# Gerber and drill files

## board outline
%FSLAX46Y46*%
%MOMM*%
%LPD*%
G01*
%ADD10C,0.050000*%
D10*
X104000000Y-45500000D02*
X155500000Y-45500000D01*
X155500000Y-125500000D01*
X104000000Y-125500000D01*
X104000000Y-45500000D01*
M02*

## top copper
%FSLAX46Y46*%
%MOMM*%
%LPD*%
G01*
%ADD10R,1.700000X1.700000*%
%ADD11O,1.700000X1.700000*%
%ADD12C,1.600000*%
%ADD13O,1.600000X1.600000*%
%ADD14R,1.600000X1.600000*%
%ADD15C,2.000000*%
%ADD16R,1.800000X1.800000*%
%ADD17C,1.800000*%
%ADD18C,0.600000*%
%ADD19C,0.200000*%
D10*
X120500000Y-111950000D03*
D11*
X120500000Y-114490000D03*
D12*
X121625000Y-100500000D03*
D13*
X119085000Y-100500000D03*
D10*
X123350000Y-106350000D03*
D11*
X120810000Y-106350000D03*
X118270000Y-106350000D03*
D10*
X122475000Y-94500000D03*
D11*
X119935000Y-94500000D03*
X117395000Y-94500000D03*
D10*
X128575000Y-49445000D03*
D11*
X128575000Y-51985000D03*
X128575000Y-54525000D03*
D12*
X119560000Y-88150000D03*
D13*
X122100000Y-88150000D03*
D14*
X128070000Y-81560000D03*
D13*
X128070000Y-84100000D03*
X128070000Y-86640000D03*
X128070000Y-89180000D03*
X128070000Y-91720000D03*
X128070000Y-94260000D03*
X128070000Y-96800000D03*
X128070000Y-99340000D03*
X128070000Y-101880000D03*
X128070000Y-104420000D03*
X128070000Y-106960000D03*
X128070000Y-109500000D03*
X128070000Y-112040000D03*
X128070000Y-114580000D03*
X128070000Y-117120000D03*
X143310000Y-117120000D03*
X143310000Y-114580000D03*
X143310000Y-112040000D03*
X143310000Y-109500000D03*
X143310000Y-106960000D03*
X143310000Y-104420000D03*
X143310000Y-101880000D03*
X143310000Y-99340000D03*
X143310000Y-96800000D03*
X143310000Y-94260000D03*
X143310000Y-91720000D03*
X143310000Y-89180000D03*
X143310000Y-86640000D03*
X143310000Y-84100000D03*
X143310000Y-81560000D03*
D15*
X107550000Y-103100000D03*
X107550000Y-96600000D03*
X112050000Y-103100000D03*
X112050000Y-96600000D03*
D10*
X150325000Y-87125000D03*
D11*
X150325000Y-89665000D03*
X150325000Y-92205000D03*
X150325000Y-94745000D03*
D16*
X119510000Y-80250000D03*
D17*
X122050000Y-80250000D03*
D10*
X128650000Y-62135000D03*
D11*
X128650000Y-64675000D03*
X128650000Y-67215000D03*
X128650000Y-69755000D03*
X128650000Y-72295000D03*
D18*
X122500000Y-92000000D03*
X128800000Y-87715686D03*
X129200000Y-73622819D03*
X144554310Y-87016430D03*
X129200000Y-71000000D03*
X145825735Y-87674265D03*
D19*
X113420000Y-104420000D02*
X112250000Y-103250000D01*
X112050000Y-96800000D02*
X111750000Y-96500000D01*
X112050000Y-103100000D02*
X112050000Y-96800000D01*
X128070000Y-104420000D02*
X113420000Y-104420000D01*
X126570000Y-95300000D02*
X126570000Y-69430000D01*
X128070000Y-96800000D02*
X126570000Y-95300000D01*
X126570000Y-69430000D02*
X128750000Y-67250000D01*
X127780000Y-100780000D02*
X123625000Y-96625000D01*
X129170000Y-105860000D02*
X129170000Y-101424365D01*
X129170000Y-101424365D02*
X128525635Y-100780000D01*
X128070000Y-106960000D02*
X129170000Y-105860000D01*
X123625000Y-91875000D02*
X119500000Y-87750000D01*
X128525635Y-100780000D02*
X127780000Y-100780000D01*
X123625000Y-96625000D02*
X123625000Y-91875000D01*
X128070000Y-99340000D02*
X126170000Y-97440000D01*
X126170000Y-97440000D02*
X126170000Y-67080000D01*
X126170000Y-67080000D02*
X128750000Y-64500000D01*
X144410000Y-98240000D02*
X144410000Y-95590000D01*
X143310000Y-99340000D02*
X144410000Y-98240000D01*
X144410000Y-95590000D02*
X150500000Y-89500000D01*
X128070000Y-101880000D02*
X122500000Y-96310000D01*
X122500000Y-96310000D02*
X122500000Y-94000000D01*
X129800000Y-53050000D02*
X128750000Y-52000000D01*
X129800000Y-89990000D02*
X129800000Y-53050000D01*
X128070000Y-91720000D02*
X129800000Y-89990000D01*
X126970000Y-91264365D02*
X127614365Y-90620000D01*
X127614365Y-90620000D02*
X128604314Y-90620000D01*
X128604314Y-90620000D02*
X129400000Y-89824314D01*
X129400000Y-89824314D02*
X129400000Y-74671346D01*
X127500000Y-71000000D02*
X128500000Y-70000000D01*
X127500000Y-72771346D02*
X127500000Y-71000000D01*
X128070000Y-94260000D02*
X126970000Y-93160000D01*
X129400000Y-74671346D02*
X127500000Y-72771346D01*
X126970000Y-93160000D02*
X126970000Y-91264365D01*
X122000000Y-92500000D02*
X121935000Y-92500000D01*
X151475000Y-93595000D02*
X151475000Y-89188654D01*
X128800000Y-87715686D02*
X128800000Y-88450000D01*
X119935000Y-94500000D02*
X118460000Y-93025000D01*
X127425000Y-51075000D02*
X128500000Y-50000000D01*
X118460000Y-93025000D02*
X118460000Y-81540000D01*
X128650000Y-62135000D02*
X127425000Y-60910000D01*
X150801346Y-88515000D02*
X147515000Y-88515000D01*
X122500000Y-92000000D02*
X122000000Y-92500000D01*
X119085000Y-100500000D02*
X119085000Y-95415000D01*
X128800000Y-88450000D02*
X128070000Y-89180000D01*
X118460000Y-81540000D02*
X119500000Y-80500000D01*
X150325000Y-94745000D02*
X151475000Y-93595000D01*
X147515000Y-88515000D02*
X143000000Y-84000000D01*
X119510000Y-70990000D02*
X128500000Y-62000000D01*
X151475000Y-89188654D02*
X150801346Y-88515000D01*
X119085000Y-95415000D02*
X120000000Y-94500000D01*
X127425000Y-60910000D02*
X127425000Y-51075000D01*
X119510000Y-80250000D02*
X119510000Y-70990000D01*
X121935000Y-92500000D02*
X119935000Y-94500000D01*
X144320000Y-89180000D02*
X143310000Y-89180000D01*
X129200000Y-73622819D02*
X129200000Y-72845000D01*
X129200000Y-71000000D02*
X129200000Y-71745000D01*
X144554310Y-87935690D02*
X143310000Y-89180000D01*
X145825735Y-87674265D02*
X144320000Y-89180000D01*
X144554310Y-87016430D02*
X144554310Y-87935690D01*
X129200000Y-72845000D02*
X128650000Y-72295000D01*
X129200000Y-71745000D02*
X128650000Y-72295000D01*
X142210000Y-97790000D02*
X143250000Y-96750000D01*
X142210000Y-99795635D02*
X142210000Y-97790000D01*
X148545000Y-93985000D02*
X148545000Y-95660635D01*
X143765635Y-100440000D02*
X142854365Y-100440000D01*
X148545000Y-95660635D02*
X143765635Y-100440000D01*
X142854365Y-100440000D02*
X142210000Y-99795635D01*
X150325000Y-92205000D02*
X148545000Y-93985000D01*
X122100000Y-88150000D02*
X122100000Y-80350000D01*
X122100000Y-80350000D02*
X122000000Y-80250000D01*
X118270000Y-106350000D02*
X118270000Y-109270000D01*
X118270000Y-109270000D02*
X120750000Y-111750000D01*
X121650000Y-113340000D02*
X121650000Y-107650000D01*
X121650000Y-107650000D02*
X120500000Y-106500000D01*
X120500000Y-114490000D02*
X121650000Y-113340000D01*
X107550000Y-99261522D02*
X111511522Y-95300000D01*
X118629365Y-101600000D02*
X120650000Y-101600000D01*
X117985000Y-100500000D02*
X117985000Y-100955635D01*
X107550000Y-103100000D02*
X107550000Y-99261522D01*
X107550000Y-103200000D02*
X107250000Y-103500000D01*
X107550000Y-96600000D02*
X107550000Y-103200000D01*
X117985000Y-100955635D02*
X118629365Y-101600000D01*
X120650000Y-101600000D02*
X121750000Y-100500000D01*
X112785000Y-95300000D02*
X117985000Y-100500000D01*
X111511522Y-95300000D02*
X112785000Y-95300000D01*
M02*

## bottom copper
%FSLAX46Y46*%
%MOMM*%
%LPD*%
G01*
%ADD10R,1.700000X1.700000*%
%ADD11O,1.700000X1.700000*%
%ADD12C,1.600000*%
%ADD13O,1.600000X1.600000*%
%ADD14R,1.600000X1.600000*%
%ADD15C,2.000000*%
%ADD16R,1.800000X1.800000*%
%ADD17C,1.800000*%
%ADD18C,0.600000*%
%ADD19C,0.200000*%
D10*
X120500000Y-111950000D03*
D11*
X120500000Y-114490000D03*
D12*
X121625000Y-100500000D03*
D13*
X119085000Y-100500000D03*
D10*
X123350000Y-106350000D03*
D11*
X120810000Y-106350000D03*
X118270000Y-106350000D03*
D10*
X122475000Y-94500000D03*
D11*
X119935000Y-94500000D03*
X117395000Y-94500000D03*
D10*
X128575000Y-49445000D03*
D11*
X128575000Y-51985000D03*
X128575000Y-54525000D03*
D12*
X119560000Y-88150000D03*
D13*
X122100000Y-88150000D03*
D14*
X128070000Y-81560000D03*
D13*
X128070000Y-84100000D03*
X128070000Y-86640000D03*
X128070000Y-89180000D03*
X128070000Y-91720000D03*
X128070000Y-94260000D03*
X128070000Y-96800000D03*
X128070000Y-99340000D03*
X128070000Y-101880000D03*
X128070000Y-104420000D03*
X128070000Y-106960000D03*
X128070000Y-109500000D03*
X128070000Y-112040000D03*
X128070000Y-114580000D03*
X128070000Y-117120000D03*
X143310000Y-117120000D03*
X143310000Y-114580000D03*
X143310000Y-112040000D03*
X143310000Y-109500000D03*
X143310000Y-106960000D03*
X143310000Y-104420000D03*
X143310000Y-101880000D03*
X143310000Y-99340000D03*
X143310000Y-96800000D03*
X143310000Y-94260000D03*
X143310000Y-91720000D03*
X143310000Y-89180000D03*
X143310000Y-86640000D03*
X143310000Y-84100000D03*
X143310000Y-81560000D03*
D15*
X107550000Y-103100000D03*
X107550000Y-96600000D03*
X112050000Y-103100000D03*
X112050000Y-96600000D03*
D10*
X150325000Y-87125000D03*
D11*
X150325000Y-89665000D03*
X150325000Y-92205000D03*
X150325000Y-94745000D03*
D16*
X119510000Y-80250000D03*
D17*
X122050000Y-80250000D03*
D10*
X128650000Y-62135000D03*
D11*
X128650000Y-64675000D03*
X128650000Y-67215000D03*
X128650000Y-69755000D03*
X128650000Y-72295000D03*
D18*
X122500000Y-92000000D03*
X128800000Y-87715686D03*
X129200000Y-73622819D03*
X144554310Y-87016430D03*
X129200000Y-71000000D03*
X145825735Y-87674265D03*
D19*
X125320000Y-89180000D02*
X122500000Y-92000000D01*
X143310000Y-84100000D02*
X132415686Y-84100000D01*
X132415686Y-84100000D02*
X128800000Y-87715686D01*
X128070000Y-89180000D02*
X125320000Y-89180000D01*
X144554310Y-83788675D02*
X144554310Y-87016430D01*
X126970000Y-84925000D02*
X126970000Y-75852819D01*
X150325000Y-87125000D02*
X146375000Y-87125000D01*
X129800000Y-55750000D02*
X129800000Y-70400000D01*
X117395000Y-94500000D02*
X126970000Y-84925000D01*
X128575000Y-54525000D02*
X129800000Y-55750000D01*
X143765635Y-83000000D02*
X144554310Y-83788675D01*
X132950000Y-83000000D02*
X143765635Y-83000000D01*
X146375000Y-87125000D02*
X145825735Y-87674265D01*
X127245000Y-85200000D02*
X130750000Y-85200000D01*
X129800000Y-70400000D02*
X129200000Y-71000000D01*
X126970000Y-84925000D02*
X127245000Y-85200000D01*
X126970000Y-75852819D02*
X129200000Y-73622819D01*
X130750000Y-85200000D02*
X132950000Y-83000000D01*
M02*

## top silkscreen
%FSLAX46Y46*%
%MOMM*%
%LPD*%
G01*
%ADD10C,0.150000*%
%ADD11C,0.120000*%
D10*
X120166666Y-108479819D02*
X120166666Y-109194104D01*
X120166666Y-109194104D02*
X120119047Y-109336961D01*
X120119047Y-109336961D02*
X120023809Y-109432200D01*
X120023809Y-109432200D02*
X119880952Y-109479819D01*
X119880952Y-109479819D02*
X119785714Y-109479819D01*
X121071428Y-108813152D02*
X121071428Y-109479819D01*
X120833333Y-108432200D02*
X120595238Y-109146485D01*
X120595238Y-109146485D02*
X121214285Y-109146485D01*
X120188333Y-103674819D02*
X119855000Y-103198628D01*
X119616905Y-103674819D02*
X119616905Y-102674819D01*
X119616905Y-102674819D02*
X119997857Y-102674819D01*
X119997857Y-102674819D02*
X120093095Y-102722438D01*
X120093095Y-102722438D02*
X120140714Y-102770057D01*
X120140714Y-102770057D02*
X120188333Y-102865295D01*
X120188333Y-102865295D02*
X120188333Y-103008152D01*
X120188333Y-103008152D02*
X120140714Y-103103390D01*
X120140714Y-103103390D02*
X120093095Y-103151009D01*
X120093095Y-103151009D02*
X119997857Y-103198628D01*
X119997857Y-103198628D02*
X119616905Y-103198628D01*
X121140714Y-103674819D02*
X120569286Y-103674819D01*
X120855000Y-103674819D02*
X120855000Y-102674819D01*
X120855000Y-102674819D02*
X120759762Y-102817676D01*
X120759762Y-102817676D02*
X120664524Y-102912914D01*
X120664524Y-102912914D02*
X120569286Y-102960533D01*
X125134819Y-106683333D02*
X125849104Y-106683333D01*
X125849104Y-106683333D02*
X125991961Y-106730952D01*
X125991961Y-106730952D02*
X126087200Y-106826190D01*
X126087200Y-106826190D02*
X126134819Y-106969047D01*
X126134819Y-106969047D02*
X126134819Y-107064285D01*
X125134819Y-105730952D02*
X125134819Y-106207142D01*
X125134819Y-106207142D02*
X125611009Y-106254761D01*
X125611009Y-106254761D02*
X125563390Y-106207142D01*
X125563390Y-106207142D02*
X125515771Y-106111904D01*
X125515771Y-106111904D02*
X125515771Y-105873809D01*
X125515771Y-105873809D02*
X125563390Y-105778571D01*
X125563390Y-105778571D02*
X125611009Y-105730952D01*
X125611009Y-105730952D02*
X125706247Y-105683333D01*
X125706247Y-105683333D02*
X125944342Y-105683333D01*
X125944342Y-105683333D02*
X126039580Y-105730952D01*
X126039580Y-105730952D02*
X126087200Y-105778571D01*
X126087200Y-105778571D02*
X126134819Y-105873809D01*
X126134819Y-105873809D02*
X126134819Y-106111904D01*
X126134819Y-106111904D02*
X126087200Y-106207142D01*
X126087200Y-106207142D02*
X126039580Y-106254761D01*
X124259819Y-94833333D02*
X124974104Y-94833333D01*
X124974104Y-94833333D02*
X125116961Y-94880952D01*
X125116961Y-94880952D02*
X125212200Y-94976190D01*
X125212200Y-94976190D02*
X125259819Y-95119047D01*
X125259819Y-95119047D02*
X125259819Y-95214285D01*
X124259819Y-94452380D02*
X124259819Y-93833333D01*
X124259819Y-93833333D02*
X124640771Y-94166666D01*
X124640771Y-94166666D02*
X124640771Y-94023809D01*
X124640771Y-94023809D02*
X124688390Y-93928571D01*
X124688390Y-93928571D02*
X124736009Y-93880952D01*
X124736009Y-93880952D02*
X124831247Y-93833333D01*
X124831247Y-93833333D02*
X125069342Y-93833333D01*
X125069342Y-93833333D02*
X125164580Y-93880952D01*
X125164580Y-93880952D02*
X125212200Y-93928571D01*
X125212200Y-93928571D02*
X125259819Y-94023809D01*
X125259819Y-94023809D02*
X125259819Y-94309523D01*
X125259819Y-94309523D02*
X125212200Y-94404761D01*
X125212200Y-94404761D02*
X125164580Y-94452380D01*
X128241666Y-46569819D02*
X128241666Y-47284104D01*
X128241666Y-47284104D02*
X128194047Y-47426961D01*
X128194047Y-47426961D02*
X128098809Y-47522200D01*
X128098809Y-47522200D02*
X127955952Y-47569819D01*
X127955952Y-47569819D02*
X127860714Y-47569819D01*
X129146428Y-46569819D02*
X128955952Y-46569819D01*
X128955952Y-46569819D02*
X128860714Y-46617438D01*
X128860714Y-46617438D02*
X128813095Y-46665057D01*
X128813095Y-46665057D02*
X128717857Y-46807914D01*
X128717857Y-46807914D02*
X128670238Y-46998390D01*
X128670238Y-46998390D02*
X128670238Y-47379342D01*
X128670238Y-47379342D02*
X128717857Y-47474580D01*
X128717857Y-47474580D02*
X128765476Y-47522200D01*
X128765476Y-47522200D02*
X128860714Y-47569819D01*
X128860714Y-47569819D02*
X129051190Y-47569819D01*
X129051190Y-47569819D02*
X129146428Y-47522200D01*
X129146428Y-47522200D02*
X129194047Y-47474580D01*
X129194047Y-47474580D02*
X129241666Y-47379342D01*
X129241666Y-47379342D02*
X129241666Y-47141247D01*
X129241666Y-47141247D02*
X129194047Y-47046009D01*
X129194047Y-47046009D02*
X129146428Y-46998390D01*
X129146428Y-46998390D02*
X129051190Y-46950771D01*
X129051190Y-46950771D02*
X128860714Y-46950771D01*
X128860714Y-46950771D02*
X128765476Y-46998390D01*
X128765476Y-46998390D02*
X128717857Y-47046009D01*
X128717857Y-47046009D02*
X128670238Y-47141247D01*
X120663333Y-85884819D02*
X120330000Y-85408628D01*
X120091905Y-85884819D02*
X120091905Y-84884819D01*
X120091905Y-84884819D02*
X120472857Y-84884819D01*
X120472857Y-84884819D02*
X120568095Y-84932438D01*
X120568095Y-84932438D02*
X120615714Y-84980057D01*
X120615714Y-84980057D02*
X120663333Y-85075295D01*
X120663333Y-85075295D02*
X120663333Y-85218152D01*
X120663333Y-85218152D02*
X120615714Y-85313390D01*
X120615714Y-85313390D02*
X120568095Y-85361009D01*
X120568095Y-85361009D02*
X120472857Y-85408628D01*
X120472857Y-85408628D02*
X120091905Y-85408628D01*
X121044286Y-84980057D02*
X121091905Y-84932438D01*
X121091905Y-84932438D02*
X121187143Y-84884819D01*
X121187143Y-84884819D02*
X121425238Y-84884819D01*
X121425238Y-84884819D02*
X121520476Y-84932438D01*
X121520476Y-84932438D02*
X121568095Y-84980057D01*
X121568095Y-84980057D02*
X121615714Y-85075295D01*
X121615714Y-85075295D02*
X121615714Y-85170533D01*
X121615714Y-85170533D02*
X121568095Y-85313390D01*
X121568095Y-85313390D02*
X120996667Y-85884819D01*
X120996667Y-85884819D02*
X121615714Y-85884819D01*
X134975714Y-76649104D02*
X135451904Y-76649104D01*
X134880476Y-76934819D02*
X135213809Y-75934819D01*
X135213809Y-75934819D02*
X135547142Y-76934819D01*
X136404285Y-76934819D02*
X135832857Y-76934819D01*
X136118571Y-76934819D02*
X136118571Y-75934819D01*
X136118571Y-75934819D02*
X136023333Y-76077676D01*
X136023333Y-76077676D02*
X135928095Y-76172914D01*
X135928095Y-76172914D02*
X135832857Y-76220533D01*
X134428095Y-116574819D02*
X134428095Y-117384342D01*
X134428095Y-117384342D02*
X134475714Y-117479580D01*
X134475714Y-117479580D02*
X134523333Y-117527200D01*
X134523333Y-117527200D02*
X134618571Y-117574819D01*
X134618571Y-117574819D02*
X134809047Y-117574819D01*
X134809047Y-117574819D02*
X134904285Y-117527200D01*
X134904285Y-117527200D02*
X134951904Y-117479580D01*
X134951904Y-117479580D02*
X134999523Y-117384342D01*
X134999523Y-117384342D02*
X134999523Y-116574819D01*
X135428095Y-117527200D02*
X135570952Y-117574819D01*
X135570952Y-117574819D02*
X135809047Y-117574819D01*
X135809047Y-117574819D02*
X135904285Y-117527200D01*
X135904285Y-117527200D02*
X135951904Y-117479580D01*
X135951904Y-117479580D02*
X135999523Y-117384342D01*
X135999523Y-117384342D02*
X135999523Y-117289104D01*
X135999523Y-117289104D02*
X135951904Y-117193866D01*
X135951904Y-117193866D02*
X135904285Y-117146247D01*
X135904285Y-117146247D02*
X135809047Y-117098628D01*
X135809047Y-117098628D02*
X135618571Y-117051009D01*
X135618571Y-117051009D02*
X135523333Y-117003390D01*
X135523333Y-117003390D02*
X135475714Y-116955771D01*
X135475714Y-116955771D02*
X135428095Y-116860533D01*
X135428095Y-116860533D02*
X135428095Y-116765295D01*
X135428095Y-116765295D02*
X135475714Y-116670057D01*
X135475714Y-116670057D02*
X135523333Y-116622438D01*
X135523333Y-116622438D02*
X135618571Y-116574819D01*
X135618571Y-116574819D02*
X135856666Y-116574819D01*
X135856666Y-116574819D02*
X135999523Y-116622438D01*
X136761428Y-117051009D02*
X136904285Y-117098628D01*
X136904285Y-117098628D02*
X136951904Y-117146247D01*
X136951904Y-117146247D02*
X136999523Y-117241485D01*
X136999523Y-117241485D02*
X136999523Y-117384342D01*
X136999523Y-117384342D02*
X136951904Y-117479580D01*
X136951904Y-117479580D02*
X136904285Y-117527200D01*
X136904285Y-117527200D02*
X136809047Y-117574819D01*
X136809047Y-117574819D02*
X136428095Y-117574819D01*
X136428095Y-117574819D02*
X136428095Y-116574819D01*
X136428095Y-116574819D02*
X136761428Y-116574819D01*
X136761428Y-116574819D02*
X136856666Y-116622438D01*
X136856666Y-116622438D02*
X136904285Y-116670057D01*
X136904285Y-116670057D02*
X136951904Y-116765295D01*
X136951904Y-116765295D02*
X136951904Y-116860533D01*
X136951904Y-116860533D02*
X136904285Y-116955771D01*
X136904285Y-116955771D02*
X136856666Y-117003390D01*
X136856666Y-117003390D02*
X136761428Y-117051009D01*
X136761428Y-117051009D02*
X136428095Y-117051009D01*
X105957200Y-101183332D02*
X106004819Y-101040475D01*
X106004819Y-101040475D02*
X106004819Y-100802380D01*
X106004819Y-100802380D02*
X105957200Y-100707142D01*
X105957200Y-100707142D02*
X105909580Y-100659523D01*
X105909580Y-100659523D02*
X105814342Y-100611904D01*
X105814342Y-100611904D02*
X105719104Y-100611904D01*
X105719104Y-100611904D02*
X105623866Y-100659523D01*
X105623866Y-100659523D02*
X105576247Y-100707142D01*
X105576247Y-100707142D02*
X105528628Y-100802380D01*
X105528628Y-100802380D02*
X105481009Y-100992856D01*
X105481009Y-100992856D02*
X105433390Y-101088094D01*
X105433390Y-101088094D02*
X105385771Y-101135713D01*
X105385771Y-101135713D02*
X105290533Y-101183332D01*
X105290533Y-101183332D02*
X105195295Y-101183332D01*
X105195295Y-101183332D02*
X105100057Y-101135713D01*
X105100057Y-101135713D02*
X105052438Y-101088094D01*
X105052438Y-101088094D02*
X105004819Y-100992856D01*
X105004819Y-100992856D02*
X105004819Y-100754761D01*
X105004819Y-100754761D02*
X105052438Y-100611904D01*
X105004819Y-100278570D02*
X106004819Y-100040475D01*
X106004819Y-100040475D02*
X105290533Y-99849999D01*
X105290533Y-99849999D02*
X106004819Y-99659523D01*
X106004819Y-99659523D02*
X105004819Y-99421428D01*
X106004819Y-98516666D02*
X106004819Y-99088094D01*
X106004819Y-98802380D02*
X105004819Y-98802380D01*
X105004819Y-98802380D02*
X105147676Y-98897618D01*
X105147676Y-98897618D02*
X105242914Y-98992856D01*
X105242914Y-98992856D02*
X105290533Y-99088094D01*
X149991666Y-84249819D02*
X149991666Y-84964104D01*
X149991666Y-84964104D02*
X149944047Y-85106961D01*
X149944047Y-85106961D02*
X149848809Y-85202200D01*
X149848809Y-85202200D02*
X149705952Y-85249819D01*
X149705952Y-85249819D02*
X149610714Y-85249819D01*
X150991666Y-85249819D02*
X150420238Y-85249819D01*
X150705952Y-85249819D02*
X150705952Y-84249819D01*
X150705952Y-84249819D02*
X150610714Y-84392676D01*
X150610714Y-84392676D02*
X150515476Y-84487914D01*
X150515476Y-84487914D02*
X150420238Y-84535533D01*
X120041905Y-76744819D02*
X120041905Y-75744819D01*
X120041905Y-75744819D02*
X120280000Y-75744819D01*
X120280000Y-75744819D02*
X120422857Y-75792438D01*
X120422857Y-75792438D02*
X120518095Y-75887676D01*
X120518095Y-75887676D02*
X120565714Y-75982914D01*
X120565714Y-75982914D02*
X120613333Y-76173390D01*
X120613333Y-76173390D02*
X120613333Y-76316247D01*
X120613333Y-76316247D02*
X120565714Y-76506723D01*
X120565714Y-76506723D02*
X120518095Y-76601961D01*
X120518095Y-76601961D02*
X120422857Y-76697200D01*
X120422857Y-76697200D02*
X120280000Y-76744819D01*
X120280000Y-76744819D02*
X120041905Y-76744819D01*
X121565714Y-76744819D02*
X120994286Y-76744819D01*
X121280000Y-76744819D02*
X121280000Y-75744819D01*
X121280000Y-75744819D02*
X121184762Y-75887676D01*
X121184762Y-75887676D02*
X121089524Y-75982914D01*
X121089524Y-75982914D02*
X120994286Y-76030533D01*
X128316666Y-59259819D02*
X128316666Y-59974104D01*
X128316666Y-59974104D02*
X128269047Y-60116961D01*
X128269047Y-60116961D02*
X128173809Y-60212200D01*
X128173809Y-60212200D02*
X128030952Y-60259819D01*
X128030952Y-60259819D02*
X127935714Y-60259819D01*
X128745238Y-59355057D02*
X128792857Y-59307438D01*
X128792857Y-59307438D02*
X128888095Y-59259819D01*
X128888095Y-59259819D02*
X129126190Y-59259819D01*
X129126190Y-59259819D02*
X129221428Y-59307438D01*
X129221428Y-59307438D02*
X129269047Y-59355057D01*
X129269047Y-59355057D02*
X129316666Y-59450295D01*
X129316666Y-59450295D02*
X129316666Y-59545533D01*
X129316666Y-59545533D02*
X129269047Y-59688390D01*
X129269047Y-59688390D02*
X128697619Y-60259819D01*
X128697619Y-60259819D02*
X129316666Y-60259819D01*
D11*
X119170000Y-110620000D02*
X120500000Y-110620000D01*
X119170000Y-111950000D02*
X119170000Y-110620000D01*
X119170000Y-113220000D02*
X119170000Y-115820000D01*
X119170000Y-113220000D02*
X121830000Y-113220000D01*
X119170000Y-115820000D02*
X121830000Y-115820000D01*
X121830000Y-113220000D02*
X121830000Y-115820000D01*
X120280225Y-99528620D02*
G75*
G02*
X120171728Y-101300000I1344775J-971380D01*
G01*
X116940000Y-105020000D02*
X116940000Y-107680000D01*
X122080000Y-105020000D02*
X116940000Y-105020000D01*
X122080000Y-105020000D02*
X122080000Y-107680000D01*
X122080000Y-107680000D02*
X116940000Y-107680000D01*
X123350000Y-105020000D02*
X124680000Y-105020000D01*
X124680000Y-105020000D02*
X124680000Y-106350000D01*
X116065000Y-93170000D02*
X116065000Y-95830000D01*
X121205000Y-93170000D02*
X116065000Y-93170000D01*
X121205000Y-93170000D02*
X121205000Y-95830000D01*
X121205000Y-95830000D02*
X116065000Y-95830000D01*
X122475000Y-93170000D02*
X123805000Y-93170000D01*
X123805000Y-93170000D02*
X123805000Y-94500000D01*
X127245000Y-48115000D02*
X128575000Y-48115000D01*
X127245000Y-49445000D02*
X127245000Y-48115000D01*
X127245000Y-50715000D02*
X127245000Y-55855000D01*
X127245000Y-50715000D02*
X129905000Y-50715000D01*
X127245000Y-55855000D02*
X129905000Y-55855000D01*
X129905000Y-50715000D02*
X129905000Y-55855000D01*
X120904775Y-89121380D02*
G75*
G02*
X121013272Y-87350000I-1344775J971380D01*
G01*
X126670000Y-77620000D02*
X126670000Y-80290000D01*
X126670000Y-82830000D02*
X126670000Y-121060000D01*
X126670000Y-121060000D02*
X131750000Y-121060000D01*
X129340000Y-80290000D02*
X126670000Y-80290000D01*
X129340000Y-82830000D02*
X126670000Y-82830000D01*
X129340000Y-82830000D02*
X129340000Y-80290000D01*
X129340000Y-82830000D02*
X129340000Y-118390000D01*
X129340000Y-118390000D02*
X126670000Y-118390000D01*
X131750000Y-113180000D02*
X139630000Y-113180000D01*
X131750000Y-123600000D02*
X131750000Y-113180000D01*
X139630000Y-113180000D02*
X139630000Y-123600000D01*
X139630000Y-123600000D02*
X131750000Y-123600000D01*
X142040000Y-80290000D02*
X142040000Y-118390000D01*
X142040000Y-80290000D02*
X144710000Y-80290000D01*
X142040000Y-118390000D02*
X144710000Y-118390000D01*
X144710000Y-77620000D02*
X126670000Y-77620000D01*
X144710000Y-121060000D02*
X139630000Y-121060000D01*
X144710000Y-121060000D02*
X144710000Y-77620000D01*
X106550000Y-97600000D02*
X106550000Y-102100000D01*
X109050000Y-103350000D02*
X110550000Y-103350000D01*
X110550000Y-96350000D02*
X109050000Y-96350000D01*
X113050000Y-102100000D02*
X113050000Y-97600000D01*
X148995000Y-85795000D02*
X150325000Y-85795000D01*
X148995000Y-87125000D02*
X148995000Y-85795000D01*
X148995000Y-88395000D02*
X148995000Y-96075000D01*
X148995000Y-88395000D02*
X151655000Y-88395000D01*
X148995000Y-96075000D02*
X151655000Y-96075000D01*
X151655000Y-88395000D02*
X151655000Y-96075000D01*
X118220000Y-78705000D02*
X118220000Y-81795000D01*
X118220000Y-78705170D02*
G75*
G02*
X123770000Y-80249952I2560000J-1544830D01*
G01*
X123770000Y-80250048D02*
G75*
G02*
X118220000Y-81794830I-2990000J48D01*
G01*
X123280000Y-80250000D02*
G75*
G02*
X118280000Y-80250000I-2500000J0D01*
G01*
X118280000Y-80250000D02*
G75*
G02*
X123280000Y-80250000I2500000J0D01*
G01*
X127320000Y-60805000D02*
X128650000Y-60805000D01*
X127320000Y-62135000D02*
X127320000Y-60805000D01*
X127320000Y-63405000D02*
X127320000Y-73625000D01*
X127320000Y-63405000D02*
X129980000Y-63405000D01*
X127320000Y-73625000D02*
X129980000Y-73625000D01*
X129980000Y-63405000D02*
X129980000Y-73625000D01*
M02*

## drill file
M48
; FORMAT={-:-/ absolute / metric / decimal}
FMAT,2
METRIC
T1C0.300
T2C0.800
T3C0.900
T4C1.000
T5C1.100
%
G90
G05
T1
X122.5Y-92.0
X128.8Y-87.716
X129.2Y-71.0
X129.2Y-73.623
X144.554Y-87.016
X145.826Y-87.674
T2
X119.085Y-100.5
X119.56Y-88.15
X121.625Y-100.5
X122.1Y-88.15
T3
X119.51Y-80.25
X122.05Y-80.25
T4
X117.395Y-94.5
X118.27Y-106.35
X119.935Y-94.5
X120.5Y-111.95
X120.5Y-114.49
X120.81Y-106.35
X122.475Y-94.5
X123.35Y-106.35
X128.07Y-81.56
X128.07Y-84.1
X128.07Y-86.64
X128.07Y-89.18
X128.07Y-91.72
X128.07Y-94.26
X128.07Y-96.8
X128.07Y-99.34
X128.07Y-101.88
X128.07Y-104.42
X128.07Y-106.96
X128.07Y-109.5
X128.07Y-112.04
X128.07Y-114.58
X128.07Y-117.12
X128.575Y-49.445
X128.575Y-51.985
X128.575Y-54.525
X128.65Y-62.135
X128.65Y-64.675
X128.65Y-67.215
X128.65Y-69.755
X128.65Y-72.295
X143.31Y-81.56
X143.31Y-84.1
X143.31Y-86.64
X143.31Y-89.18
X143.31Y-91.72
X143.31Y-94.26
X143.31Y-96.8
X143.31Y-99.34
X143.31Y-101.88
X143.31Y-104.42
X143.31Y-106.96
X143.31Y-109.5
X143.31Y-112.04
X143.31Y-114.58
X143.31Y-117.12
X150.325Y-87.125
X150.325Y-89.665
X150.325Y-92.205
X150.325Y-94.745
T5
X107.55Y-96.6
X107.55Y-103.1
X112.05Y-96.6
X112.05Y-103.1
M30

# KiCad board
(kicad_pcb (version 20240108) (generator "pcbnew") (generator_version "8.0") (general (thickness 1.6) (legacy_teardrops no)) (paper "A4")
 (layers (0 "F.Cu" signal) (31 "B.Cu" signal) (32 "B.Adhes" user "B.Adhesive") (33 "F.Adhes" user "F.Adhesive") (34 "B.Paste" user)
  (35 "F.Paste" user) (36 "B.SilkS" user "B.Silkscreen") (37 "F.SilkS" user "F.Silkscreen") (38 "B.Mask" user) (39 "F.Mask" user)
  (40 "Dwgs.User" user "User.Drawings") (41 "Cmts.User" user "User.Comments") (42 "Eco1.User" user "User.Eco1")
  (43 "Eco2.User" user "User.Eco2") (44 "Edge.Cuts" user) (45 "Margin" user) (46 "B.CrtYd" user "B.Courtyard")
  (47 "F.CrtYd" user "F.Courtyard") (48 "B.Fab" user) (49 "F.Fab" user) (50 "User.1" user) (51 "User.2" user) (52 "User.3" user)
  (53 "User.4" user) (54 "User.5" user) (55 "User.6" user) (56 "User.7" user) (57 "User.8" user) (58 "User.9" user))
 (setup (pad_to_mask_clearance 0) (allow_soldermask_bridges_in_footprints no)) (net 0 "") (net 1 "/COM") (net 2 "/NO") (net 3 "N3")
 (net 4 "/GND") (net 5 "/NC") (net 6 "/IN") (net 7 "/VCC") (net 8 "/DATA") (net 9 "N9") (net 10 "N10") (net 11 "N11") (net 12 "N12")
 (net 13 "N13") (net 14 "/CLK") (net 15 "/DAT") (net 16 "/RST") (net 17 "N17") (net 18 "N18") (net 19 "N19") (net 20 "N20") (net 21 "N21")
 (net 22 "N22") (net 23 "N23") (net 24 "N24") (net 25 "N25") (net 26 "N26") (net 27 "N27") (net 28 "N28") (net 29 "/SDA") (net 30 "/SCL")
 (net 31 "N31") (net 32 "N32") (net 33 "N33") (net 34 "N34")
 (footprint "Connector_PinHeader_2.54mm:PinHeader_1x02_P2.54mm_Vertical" (layer "F.Cu") (at 120.5 111.95)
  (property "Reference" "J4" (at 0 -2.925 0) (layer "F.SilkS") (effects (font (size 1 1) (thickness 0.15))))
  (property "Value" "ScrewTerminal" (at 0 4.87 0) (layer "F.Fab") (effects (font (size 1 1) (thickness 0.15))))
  (fp_line (start -1.33 -1.33) (end 0 -1.33) (stroke (width 0.12) (type solid)) (layer "F.SilkS"))
  (fp_line (start -1.33 0) (end -1.33 -1.33) (stroke (width 0.12) (type solid)) (layer "F.SilkS"))
  (fp_line (start -1.33 1.27) (end -1.33 3.87) (stroke (width 0.12) (type solid)) (layer "F.SilkS"))
  (fp_line (start -1.33 1.27) (end 1.33 1.27) (stroke (width 0.12) (type solid)) (layer "F.SilkS"))
  (fp_line (start -1.33 3.87) (end 1.33 3.87) (stroke (width 0.12) (type solid)) (layer "F.SilkS"))
  (fp_line (start 1.33 1.27) (end 1.33 3.87) (stroke (width 0.12) (type solid)) (layer "F.SilkS"))
  (pad "1" thru_hole rect (at 0 0) (size 1.7 1.7) (drill 1) (layers "*.Cu" "*.Mask") (remove_unused_layers no) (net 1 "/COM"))
  (pad "2" thru_hole oval (at 0 2.54) (size 1.7 1.7) (drill 1) (layers "*.Cu" "*.Mask") (remove_unused_layers no) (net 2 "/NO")))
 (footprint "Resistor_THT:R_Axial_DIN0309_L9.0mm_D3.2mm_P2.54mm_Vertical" (layer "F.Cu") (at 121.625 100.5 180)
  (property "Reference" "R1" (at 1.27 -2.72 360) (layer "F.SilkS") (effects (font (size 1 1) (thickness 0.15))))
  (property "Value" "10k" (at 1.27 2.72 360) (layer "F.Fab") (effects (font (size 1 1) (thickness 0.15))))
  (fp_arc (start 1.344775 0.97138) (mid -1.655812 -0.101418) (end 1.453272 -0.8) (stroke (width 0.12) (type solid)) (layer "F.SilkS"))
  (pad "1" thru_hole circle (at 0 0 180) (size 1.6 1.6) (drill 0.8) (layers "*.Cu" "*.Mask") (remove_unused_layers no) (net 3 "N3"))
  (pad "2" thru_hole oval (at 2.54 0 180) (size 1.6 1.6) (drill 0.8) (layers "*.Cu" "*.Mask") (remove_unused_layers no) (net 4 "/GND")))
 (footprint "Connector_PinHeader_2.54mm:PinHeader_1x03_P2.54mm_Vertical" (layer "F.Cu") (at 123.35 106.35 -90)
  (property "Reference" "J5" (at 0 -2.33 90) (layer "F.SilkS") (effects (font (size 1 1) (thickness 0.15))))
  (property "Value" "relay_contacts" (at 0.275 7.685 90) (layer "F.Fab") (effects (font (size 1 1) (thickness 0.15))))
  (fp_line (start -1.33 6.41) (end 1.33 6.41) (stroke (width 0.12) (type solid)) (layer "F.SilkS"))
  (fp_line (start -1.33 1.27) (end -1.33 6.41) (stroke (width 0.12) (type solid)) (layer "F.SilkS"))
  (fp_line (start -1.33 1.27) (end 1.33 1.27) (stroke (width 0.12) (type solid)) (layer "F.SilkS"))
  (fp_line (start 1.33 1.27) (end 1.33 6.41) (stroke (width 0.12) (type solid)) (layer "F.SilkS"))
  (fp_line (start -1.33 0) (end -1.33 -1.33) (stroke (width 0.12) (type solid)) (layer "F.SilkS"))
  (fp_line (start -1.33 -1.33) (end 0 -1.33) (stroke (width 0.12) (type solid)) (layer "F.SilkS"))
  (pad "1" thru_hole rect (at 0 0 270) (size 1.7 1.7) (drill 1) (layers "*.Cu" "*.Mask") (remove_unused_layers no) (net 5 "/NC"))
  (pad "2" thru_hole oval (at 0 2.54 270) (size 1.7 1.7) (drill 1) (layers "*.Cu" "*.Mask") (remove_unused_layers no) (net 2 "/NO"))
  (pad "3" thru_hole oval (at 0 5.08 270) (size 1.7 1.7) (drill 1) (layers "*.Cu" "*.Mask") (remove_unused_layers no) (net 1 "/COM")))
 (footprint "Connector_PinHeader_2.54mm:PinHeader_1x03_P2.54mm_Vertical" (layer "F.Cu") (at 122.475 94.5 -90)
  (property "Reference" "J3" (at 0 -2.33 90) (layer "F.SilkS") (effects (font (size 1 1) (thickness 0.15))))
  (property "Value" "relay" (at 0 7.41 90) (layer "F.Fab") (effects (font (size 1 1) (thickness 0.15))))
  (fp_line (start -1.33 6.41) (end 1.33 6.41) (stroke (width 0.12) (type solid)) (layer "F.SilkS"))
  (fp_line (start -1.33 1.27) (end -1.33 6.41) (stroke (width 0.12) (type solid)) (layer "F.SilkS"))
  (fp_line (start -1.33 1.27) (end 1.33 1.27) (stroke (width 0.12) (type solid)) (layer "F.SilkS"))
  (fp_line (start 1.33 1.27) (end 1.33 6.41) (stroke (width 0.12) (type solid)) (layer "F.SilkS"))
  (fp_line (start -1.33 0) (end -1.33 -1.33) (stroke (width 0.12) (type solid)) (layer "F.SilkS"))
  (fp_line (start -1.33 -1.33) (end 0 -1.33) (stroke (width 0.12) (type solid)) (layer "F.SilkS"))
  (pad "1" thru_hole rect (at 0 0 270) (size 1.7 1.7) (drill 1) (layers "*.Cu" "*.Mask") (remove_unused_layers no) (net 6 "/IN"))
  (pad "2" thru_hole oval (at 0 2.54 270) (size 1.7 1.7) (drill 1) (layers "*.Cu" "*.Mask") (remove_unused_layers no) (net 4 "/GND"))
  (pad "3" thru_hole oval (at 0 5.08 270) (size 1.7 1.7) (drill 1) (layers "*.Cu" "*.Mask") (remove_unused_layers no) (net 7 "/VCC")))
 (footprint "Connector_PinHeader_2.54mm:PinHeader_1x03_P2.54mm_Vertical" (layer "F.Cu") (at 128.575 49.445)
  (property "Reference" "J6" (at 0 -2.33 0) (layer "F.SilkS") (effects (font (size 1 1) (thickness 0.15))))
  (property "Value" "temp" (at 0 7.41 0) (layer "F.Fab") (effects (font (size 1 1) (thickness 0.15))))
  (fp_line (start -1.33 -1.33) (end 0 -1.33) (stroke (width 0.12) (type solid)) (layer "F.SilkS"))
  (fp_line (start -1.33 0) (end -1.33 -1.33) (stroke (width 0.12) (type solid)) (layer "F.SilkS"))
  (fp_line (start -1.33 1.27) (end -1.33 6.41) (stroke (width 0.12) (type solid)) (layer "F.SilkS"))
  (fp_line (start -1.33 1.27) (end 1.33 1.27) (stroke (width 0.12) (type solid)) (layer "F.SilkS"))
  (fp_line (start -1.33 6.41) (end 1.33 6.41) (stroke (width 0.12) (type solid)) (layer "F.SilkS"))
  (fp_line (start 1.33 1.27) (end 1.33 6.41) (stroke (width 0.12) (type solid)) (layer "F.SilkS"))
  (pad "1" thru_hole rect (at 0 0) (size 1.7 1.7) (drill 1) (layers "*.Cu" "*.Mask") (remove_unused_layers no) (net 4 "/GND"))
  (pad "2" thru_hole oval (at 0 2.54) (size 1.7 1.7) (drill 1) (layers "*.Cu" "*.Mask") (remove_unused_layers no) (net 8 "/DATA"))
  (pad "3" thru_hole oval (at 0 5.08) (size 1.7 1.7) (drill 1) (layers "*.Cu" "*.Mask") (remove_unused_layers no) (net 7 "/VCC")))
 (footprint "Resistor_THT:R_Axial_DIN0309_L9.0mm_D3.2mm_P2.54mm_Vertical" (layer "F.Cu") (at 119.56 88.15)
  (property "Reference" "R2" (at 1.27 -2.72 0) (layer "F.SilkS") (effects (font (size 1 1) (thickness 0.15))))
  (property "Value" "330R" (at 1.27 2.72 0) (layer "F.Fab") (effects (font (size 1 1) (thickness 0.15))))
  (fp_arc (start 1.344775 0.97138) (mid -1.655812 -0.101418) (end 1.453272 -0.8) (stroke (width 0.12) (type solid)) (layer "F.SilkS"))
  (pad "1" thru_hole circle (at 0 0) (size 1.6 1.6) (drill 0.8) (layers "*.Cu" "*.Mask") (remove_unused_layers no) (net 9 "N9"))
  (pad "2" thru_hole oval (at 2.54 0) (size 1.6 1.6) (drill 0.8) (layers "*.Cu" "*.Mask") (remove_unused_layers no) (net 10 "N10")))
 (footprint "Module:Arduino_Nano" (layer "F.Cu") (at 128.07 81.56)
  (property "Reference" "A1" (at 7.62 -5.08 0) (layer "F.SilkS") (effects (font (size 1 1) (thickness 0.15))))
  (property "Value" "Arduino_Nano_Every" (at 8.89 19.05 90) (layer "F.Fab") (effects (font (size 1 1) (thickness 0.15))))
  (fp_line (start -1.4 -3.94) (end -1.4 -1.27) (stroke (width 0.12) (type solid)) (layer "F.SilkS"))
  (fp_line (start -1.4 1.27) (end -1.4 39.5) (stroke (width 0.12) (type solid)) (layer "F.SilkS"))
  (fp_line (start -1.4 39.5) (end 3.68 39.5) (stroke (width 0.12) (type solid)) (layer "F.SilkS"))
  (fp_line (start 1.27 -1.27) (end -1.4 -1.27) (stroke (width 0.12) (type solid)) (layer "F.SilkS"))
  (fp_line (start 1.27 1.27) (end -1.4 1.27) (stroke (width 0.12) (type solid)) (layer "F.SilkS"))
  (fp_line (start 1.27 1.27) (end 1.27 -1.27) (stroke (width 0.12) (type solid)) (layer "F.SilkS"))
  (fp_line (start 1.27 1.27) (end 1.27 36.83) (stroke (width 0.12) (type solid)) (layer "F.SilkS"))
  (fp_line (start 1.27 36.83) (end -1.4 36.83) (stroke (width 0.12) (type solid)) (layer "F.SilkS"))
  (fp_line (start 3.68 31.62) (end 11.56 31.62) (stroke (width 0.12) (type solid)) (layer "F.SilkS"))
  (fp_line (start 3.68 42.04) (end 3.68 31.62) (stroke (width 0.12) (type solid)) (layer "F.SilkS"))
  (fp_line (start 11.56 31.62) (end 11.56 42.04) (stroke (width 0.12) (type solid)) (layer "F.SilkS"))
  (fp_line (start 11.56 42.04) (end 3.68 42.04) (stroke (width 0.12) (type solid)) (layer "F.SilkS"))
  (fp_line (start 13.97 -1.27) (end 13.97 36.83) (stroke (width 0.12) (type solid)) (layer "F.SilkS"))
  (fp_line (start 13.97 -1.27) (end 16.64 -1.27) (stroke (width 0.12) (type solid)) (layer "F.SilkS"))
  (fp_line (start 13.97 36.83) (end 16.64 36.83) (stroke (width 0.12) (type solid)) (layer "F.SilkS"))
  (fp_line (start 16.64 -3.94) (end -1.4 -3.94) (stroke (width 0.12) (type solid)) (layer "F.SilkS"))
  (fp_line (start 16.64 39.5) (end 11.56 39.5) (stroke (width 0.12) (type solid)) (layer "F.SilkS"))
  (fp_line (start 16.64 39.5) (end 16.64 -3.94) (stroke (width 0.12) (type solid)) (layer "F.SilkS"))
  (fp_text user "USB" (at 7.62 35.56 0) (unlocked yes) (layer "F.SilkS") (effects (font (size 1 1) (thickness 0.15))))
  (pad "1" thru_hole rect (at 0 0) (size 1.6 1.6) (drill 1) (layers "*.Cu" "*.Mask") (remove_unused_layers no) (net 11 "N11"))
  (pad "2" thru_hole oval (at 0 2.54) (size 1.6 1.6) (drill 1) (layers "*.Cu" "*.Mask") (remove_unused_layers no) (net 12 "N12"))
  (pad "3" thru_hole oval (at 0 5.08) (size 1.6 1.6) (drill 1) (layers "*.Cu" "*.Mask") (remove_unused_layers no) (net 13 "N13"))
  (pad "4" thru_hole oval (at 0 7.62) (size 1.6 1.6) (drill 1) (layers "*.Cu" "*.Mask") (remove_unused_layers no) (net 4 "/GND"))
  (pad "5" thru_hole oval (at 0 10.16) (size 1.6 1.6) (drill 1) (layers "*.Cu" "*.Mask") (remove_unused_layers no) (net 8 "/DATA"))
  (pad "6" thru_hole oval (at 0 12.7) (size 1.6 1.6) (drill 1) (layers "*.Cu" "*.Mask") (remove_unused_layers no) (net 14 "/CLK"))
  (pad "7" thru_hole oval (at 0 15.24) (size 1.6 1.6) (drill 1) (layers "*.Cu" "*.Mask") (remove_unused_layers no) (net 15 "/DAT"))
  (pad "8" thru_hole oval (at 0 17.78) (size 1.6 1.6) (drill 1) (layers "*.Cu" "*.Mask") (remove_unused_layers no) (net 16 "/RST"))
  (pad "9" thru_hole oval (at 0 20.32) (size 1.6 1.6) (drill 1) (layers "*.Cu" "*.Mask") (remove_unused_layers no) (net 6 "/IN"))
  (pad "10" thru_hole oval (at 0 22.86) (size 1.6 1.6) (drill 1) (layers "*.Cu" "*.Mask") (remove_unused_layers no) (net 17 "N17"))
  (pad "11" thru_hole oval (at 0 25.4) (size 1.6 1.6) (drill 1) (layers "*.Cu" "*.Mask") (remove_unused_layers no) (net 9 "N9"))
  (pad "12" thru_hole oval (at 0 27.94) (size 1.6 1.6) (drill 1) (layers "*.Cu" "*.Mask") (remove_unused_layers no) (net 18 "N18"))
  (pad "13" thru_hole oval (at 0 30.48) (size 1.6 1.6) (drill 1) (layers "*.Cu" "*.Mask") (remove_unused_layers no) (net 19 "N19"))
  (pad "14" thru_hole oval (at 0 33.02) (size 1.6 1.6) (drill 1) (layers "*.Cu" "*.Mask") (remove_unused_layers no) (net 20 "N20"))
  (pad "15" thru_hole oval (at 0 35.56) (size 1.6 1.6) (drill 1) (layers "*.Cu" "*.Mask") (remove_unused_layers no) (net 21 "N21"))
  (pad "16" thru_hole oval (at 15.24 35.56) (size 1.6 1.6) (drill 1) (layers "*.Cu" "*.Mask") (remove_unused_layers no) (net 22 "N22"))
  (pad "17" thru_hole oval (at 15.24 33.02) (size 1.6 1.6) (drill 1) (layers "*.Cu" "*.Mask") (remove_unused_layers no) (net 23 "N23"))
  (pad "18" thru_hole oval (at 15.24 30.48) (size 1.6 1.6) (drill 1) (layers "*.Cu" "*.Mask") (remove_unused_layers no) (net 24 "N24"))
  (pad "19" thru_hole oval (at 15.24 27.94) (size 1.6 1.6) (drill 1) (layers "*.Cu" "*.Mask") (remove_unused_layers no) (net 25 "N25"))
  (pad "20" thru_hole oval (at 15.24 25.4) (size 1.6 1.6) (drill 1) (layers "*.Cu" "*.Mask") (remove_unused_layers no) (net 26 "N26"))
  (pad "21" thru_hole oval (at 15.24 22.86) (size 1.6 1.6) (drill 1) (layers "*.Cu" "*.Mask") (remove_unused_layers no) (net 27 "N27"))
  (pad "22" thru_hole oval (at 15.24 20.32) (size 1.6 1.6) (drill 1) (layers "*.Cu" "*.Mask") (remove_unused_layers no) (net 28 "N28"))
  (pad "23" thru_hole oval (at 15.24 17.78) (size 1.6 1.6) (drill 1) (layers "*.Cu" "*.Mask") (remove_unused_layers no) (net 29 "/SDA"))
  (pad "24" thru_hole oval (at 15.24 15.24) (size 1.6 1.6) (drill 1) (layers "*.Cu" "*.Mask") (remove_unused_layers no) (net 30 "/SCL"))
  (pad "25" thru_hole oval (at 15.24 12.7) (size 1.6 1.6) (drill 1) (layers "*.Cu" "*.Mask") (remove_unused_layers no) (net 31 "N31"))
  (pad "26" thru_hole oval (at 15.24 10.16) (size 1.6 1.6) (drill 1) (layers "*.Cu" "*.Mask") (remove_unused_layers no) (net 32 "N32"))
  (pad "27" thru_hole oval (at 15.24 7.62) (size 1.6 1.6) (drill 1) (layers "*.Cu" "*.Mask") (remove_unused_layers no) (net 7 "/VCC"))
  (pad "28" thru_hole oval (at 15.24 5.08) (size 1.6 1.6) (drill 1) (layers "*.Cu" "*.Mask") (remove_unused_layers no) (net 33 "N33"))
  (pad "29" thru_hole oval (at 15.24 2.54) (size 1.6 1.6) (drill 1) (layers "*.Cu" "*.Mask") (remove_unused_layers no) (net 4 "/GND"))
  (pad "30" thru_hole oval (at 15.24 0) (size 1.6 1.6) (drill 1) (layers "*.Cu" "*.Mask") (remove_unused_layers no) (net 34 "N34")))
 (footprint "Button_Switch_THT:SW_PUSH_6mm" (layer "F.Cu") (at 107.55 103.1 90)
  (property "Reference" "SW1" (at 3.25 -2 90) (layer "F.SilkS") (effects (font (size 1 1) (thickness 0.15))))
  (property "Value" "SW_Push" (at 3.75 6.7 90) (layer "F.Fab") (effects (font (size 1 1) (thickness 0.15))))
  (fp_line (start 5.5 -1) (end 1 -1) (stroke (width 0.12) (type solid)) (layer "F.SilkS"))
  (fp_line (start -0.25 1.5) (end -0.25 3) (stroke (width 0.12) (type solid)) (layer "F.SilkS"))
  (fp_line (start 6.75 3) (end 6.75 1.5) (stroke (width 0.12) (type solid)) (layer "F.SilkS"))
  (fp_line (start 1 5.5) (end 5.5 5.5) (stroke (width 0.12) (type solid)) (layer "F.SilkS"))
  (pad "1" thru_hole circle (at 0 0 180) (size 2 2) (drill 1.1) (layers "*.Cu" "*.Mask") (remove_unused_layers no) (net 3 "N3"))
  (pad "1" thru_hole circle (at 6.5 0 180) (size 2 2) (drill 1.1) (layers "*.Cu" "*.Mask") (remove_unused_layers no) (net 3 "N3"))
  (pad "2" thru_hole circle (at 0 4.5 180) (size 2 2) (drill 1.1) (layers "*.Cu" "*.Mask") (remove_unused_layers no) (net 17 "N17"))
  (pad "2" thru_hole circle (at 6.5 4.5 180) (size 2 2) (drill 1.1) (layers "*.Cu" "*.Mask") (remove_unused_layers no) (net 17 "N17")))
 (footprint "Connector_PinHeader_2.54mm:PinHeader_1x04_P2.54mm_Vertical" (layer "F.Cu") (at 150.325 87.125)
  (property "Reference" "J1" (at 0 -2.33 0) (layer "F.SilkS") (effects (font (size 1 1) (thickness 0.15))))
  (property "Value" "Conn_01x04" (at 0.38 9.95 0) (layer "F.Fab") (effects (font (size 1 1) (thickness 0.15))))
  (fp_line (start -1.33 -1.33) (end 0 -1.33) (stroke (width 0.12) (type solid)) (layer "F.SilkS"))
  (fp_line (start -1.33 0) (end -1.33 -1.33) (stroke (width 0.12) (type solid)) (layer "F.SilkS"))
  (fp_line (start -1.33 1.27) (end -1.33 8.95) (stroke (width 0.12) (type solid)) (layer "F.SilkS"))
  (fp_line (start -1.33 1.27) (end 1.33 1.27) (stroke (width 0.12) (type solid)) (layer "F.SilkS"))
  (fp_line (start -1.33 8.95) (end 1.33 8.95) (stroke (width 0.12) (type solid)) (layer "F.SilkS"))
  (fp_line (start 1.33 1.27) (end 1.33 8.95) (stroke (width 0.12) (type solid)) (layer "F.SilkS"))
  (pad "1" thru_hole rect (at 0 0) (size 1.7 1.7) (drill 1) (layers "*.Cu" "*.Mask") (remove_unused_layers no) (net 7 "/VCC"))
  (pad "2" thru_hole oval (at 0 2.54) (size 1.7 1.7) (drill 1) (layers "*.Cu" "*.Mask") (remove_unused_layers no) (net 29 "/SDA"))
  (pad "3" thru_hole oval (at 0 5.08) (size 1.7 1.7) (drill 1) (layers "*.Cu" "*.Mask") (remove_unused_layers no) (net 30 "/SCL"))
  (pad "4" thru_hole oval (at 0 7.62) (size 1.7 1.7) (drill 1) (layers "*.Cu" "*.Mask") (remove_unused_layers no) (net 4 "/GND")))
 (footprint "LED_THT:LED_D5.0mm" (layer "F.Cu") (at 119.51 80.25)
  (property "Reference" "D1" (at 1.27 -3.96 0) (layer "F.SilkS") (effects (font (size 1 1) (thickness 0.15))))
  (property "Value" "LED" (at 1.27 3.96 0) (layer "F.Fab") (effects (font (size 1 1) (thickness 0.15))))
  (fp_line (start -1.29 -1.545) (end -1.29 1.545) (stroke (width 0.12) (type solid)) (layer "F.SilkS"))
  (fp_arc (start -1.29 -1.54483) (mid 2.071756 -2.880501) (end 4.26 -0.000048) (stroke (width 0.12) (type solid)) (layer "F.SilkS"))
  (fp_arc (start 4.26 0.000048) (mid 2.071756 2.880501) (end -1.29 1.54483) (stroke (width 0.12) (type solid)) (layer "F.SilkS"))
  (fp_circle (center 1.27 0) (end 3.77 0) (stroke (width 0.12) (type solid)) (fill none) (layer "F.SilkS"))
  (pad "1" thru_hole rect (at 0 0) (size 1.8 1.8) (drill 0.9) (layers "*.Cu" "*.Mask") (remove_unused_layers no) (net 4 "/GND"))
  (pad "2" thru_hole circle (at 2.54 0) (size 1.8 1.8) (drill 0.9) (layers "*.Cu" "*.Mask") (remove_unused_layers no) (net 10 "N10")))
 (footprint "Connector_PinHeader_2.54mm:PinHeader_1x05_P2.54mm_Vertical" (layer "F.Cu") (at 128.65 62.135)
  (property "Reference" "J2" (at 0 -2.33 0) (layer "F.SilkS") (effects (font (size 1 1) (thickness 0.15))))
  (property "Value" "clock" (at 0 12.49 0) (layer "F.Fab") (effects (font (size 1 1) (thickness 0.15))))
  (fp_line (start -1.33 -1.33) (end 0 -1.33) (stroke (width 0.12) (type solid)) (layer "F.SilkS"))
  (fp_line (start -1.33 0) (end -1.33 -1.33) (stroke (width 0.12) (type solid)) (layer "F.SilkS"))
  (fp_line (start -1.33 1.27) (end -1.33 11.49) (stroke (width 0.12) (type solid)) (layer "F.SilkS"))
  (fp_line (start -1.33 1.27) (end 1.33 1.27) (stroke (width 0.12) (type solid)) (layer "F.SilkS"))
  (fp_line (start -1.33 11.49) (end 1.33 11.49) (stroke (width 0.12) (type solid)) (layer "F.SilkS"))
  (fp_line (start 1.33 1.27) (end 1.33 11.49) (stroke (width 0.12) (type solid)) (layer "F.SilkS"))
  (pad "1" thru_hole rect (at 0 0) (size 1.7 1.7) (drill 1) (layers "*.Cu" "*.Mask") (remove_unused_layers no) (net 4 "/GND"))
  (pad "2" thru_hole oval (at 0 2.54) (size 1.7 1.7) (drill 1) (layers "*.Cu" "*.Mask") (remove_unused_layers no) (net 16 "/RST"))
  (pad "3" thru_hole oval (at 0 5.08) (size 1.7 1.7) (drill 1) (layers "*.Cu" "*.Mask") (remove_unused_layers no) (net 15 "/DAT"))
  (pad "4" thru_hole oval (at 0 7.62) (size 1.7 1.7) (drill 1) (layers "*.Cu" "*.Mask") (remove_unused_layers no) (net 14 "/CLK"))
  (pad "5" thru_hole oval (at 0 10.16) (size 1.7 1.7) (drill 1) (layers "*.Cu" "*.Mask") (remove_unused_layers no) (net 7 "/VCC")))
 (gr_rect (start 104 45.5) (end 155.5 125.5) (stroke (width 0.05) (type default)) (fill none) (layer "Edge.Cuts"))
 (segment (start 113.42 104.42) (end 112.25 103.25) (width 0.2) (layer "F.Cu") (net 17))
 (segment (start 112.05 96.8) (end 111.75 96.5) (width 0.2) (layer "F.Cu") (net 17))
 (segment (start 112.05 103.1) (end 112.05 96.8) (width 0.2) (layer "F.Cu") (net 17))
 (segment (start 128.07 104.42) (end 113.42 104.42) (width 0.2) (layer "F.Cu") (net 17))
 (segment (start 126.57 95.3) (end 126.57 69.43) (width 0.2) (layer "F.Cu") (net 15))
 (segment (start 128.07 96.8) (end 126.57 95.3) (width 0.2) (layer "F.Cu") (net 15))
 (segment (start 126.57 69.43) (end 128.75 67.25) (width 0.2) (layer "F.Cu") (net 15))
 (segment (start 127.78 100.78) (end 123.625 96.625) (width 0.2) (layer "F.Cu") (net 9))
 (segment (start 129.17 105.86) (end 129.17 101.424365) (width 0.2) (layer "F.Cu") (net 9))
 (segment (start 129.17 101.424365) (end 128.525635 100.78) (width 0.2) (layer "F.Cu") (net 9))
 (segment (start 128.07 106.96) (end 129.17 105.86) (width 0.2) (layer "F.Cu") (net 9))
 (segment (start 123.625 91.875) (end 119.5 87.75) (width 0.2) (layer "F.Cu") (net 9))
 (segment (start 128.525635 100.78) (end 127.78 100.78) (width 0.2) (layer "F.Cu") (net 9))
 (segment (start 123.625 96.625) (end 123.625 91.875) (width 0.2) (layer "F.Cu") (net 9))
 (segment (start 128.07 99.34) (end 126.17 97.44) (width 0.2) (layer "F.Cu") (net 16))
 (segment (start 126.17 97.44) (end 126.17 67.08) (width 0.2) (layer "F.Cu") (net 16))
 (segment (start 126.17 67.08) (end 128.75 64.5) (width 0.2) (layer "F.Cu") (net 16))
 (segment (start 144.41 98.24) (end 144.41 95.59) (width 0.2) (layer "F.Cu") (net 29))
 (segment (start 143.31 99.34) (end 144.41 98.24) (width 0.2) (layer "F.Cu") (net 29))
 (segment (start 144.41 95.59) (end 150.5 89.5) (width 0.2) (layer "F.Cu") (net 29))
 (segment (start 128.07 101.88) (end 122.5 96.31) (width 0.2) (layer "F.Cu") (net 6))
 (segment (start 122.5 96.31) (end 122.5 94) (width 0.2) (layer "F.Cu") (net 6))
 (segment (start 129.8 53.05) (end 128.75 52) (width 0.2) (layer "F.Cu") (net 8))
 (segment (start 129.8 89.99) (end 129.8 53.05) (width 0.2) (layer "F.Cu") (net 8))
 (segment (start 128.07 91.72) (end 129.8 89.99) (width 0.2) (layer "F.Cu") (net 8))
 (segment (start 126.97 91.264365) (end 127.614365 90.62) (width 0.2) (layer "F.Cu") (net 14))
 (segment (start 127.614365 90.62) (end 128.604314 90.62) (width 0.2) (layer "F.Cu") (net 14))
 (segment (start 128.604314 90.62) (end 129.4 89.824314) (width 0.2) (layer "F.Cu") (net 14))
 (segment (start 129.4 89.824314) (end 129.4 74.671346) (width 0.2) (layer "F.Cu") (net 14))
 (segment (start 127.5 71) (end 128.5 70) (width 0.2) (layer "F.Cu") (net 14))
 (segment (start 127.5 72.771346) (end 127.5 71) (width 0.2) (layer "F.Cu") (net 14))
 (segment (start 128.07 94.26) (end 126.97 93.16) (width 0.2) (layer "F.Cu") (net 14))
 (segment (start 129.4 74.671346) (end 127.5 72.771346) (width 0.2) (layer "F.Cu") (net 14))
 (segment (start 126.97 93.16) (end 126.97 91.264365) (width 0.2) (layer "F.Cu") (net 14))
 (segment (start 122 92.5) (end 121.935 92.5) (width 0.2) (layer "F.Cu") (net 4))
 (segment (start 151.475 93.595) (end 151.475 89.188654) (width 0.2) (layer "F.Cu") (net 4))
 (segment (start 128.8 87.715686) (end 128.8 88.45) (width 0.2) (layer "F.Cu") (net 4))
 (segment (start 119.935 94.5) (end 118.46 93.025) (width 0.2) (layer "F.Cu") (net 4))
 (segment (start 127.425 51.075) (end 128.5 50) (width 0.2) (layer "F.Cu") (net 4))
 (segment (start 118.46 93.025) (end 118.46 81.54) (width 0.2) (layer "F.Cu") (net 4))
 (segment (start 128.65 62.135) (end 127.425 60.91) (width 0.2) (layer "F.Cu") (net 4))
 (segment (start 150.801346 88.515) (end 147.515 88.515) (width 0.2) (layer "F.Cu") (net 4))
 (segment (start 122.5 92) (end 122 92.5) (width 0.2) (layer "F.Cu") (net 4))
 (segment (start 119.085 100.5) (end 119.085 95.415) (width 0.2) (layer "F.Cu") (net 4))
 (segment (start 128.8 88.45) (end 128.07 89.18) (width 0.2) (layer "F.Cu") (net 4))
 (segment (start 118.46 81.54) (end 119.5 80.5) (width 0.2) (layer "F.Cu") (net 4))
 (segment (start 150.325 94.745) (end 151.475 93.595) (width 0.2) (layer "F.Cu") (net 4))
 (segment (start 147.515 88.515) (end 143 84) (width 0.2) (layer "F.Cu") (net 4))
 (segment (start 119.51 70.99) (end 128.5 62) (width 0.2) (layer "F.Cu") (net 4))
 (segment (start 151.475 89.188654) (end 150.801346 88.515) (width 0.2) (layer "F.Cu") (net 4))
 (segment (start 119.085 95.415) (end 120 94.5) (width 0.2) (layer "F.Cu") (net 4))
 (segment (start 127.425 60.91) (end 127.425 51.075) (width 0.2) (layer "F.Cu") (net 4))
 (segment (start 119.51 80.25) (end 119.51 70.99) (width 0.2) (layer "F.Cu") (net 4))
 (segment (start 121.935 92.5) (end 119.935 94.5) (width 0.2) (layer "F.Cu") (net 4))
 (via (at 122.5 92) (size 0.6) (drill 0.3) (layers "F.Cu" "B.Cu") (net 4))
 (via (at 128.8 87.715686) (size 0.6) (drill 0.3) (layers "F.Cu" "B.Cu") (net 4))
 (segment (start 125.32 89.18) (end 122.5 92) (width 0.2) (layer "B.Cu") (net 4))
 (segment (start 143.31 84.1) (end 132.415686 84.1) (width 0.2) (layer "B.Cu") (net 4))
 (segment (start 132.415686 84.1) (end 128.8 87.715686) (width 0.2) (layer "B.Cu") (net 4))
 (segment (start 128.07 89.18) (end 125.32 89.18) (width 0.2) (layer "B.Cu") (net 4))
 (segment (start 144.32 89.18) (end 143.31 89.18) (width 0.2) (layer "F.Cu") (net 7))
 (segment (start 129.2 73.622819) (end 129.2 72.845) (width 0.2) (layer "F.Cu") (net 7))
 (segment (start 129.2 71) (end 129.2 71.745) (width 0.2) (layer "F.Cu") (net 7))
 (segment (start 144.55431 87.93569) (end 143.31 89.18) (width 0.2) (layer "F.Cu") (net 7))
 (segment (start 145.825735 87.674265) (end 144.32 89.18) (width 0.2) (layer "F.Cu") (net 7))
 (segment (start 144.55431 87.01643) (end 144.55431 87.93569) (width 0.2) (layer "F.Cu") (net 7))
 (segment (start 129.2 72.845) (end 128.65 72.295) (width 0.2) (layer "F.Cu") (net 7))
 (segment (start 129.2 71.745) (end 128.65 72.295) (width 0.2) (layer "F.Cu") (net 7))
 (via (at 129.2 73.622819) (size 0.6) (drill 0.3) (layers "F.Cu" "B.Cu") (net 7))
 (via (at 144.55431 87.01643) (size 0.6) (drill 0.3) (layers "F.Cu" "B.Cu") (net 7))
 (via (at 129.2 71) (size 0.6) (drill 0.3) (layers "F.Cu" "B.Cu") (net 7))
 (via (at 145.825735 87.674265) (size 0.6) (drill 0.3) (layers "F.Cu" "B.Cu") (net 7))
 (segment (start 144.55431 83.788675) (end 144.55431 87.01643) (width 0.2) (layer "B.Cu") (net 7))
 (segment (start 126.97 84.925) (end 126.97 75.852819) (width 0.2) (layer "B.Cu") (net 7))
 (segment (start 150.325 87.125) (end 146.375 87.125) (width 0.2) (layer "B.Cu") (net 7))
 (segment (start 129.8 55.75) (end 129.8 70.4) (width 0.2) (layer "B.Cu") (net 7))
 (segment (start 117.395 94.5) (end 126.97 84.925) (width 0.2) (layer "B.Cu") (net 7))
 (segment (start 128.575 54.525) (end 129.8 55.75) (width 0.2) (layer "B.Cu") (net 7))
 (segment (start 143.765635 83) (end 144.55431 83.788675) (width 0.2) (layer "B.Cu") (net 7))
 (segment (start 132.95 83) (end 143.765635 83) (width 0.2) (layer "B.Cu") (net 7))
 (segment (start 146.375 87.125) (end 145.825735 87.674265) (width 0.2) (layer "B.Cu") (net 7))
 (segment (start 127.245 85.2) (end 130.75 85.2) (width 0.2) (layer "B.Cu") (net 7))
 (segment (start 129.8 70.4) (end 129.2 71) (width 0.2) (layer "B.Cu") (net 7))
 (segment (start 126.97 84.925) (end 127.245 85.2) (width 0.2) (layer "B.Cu") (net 7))
 (segment (start 126.97 75.852819) (end 129.2 73.622819) (width 0.2) (layer "B.Cu") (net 7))
 (segment (start 130.75 85.2) (end 132.95 83) (width 0.2) (layer "B.Cu") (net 7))
 (segment (start 142.21 97.79) (end 143.25 96.75) (width 0.2) (layer "F.Cu") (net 30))
 (segment (start 142.21 99.795635) (end 142.21 97.79) (width 0.2) (layer "F.Cu") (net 30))
 (segment (start 148.545 93.985) (end 148.545 95.660635) (width 0.2) (layer "F.Cu") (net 30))
 (segment (start 143.765635 100.44) (end 142.854365 100.44) (width 0.2) (layer "F.Cu") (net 30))
 (segment (start 148.545 95.660635) (end 143.765635 100.44) (width 0.2) (layer "F.Cu") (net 30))
 (segment (start 142.854365 100.44) (end 142.21 99.795635) (width 0.2) (layer "F.Cu") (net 30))
 (segment (start 150.325 92.205) (end 148.545 93.985) (width 0.2) (layer "F.Cu") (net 30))
 (segment (start 122.1 88.15) (end 122.1 80.35) (width 0.2) (layer "F.Cu") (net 10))
 (segment (start 122.1 80.35) (end 122 80.25) (width 0.2) (layer "F.Cu") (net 10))
 (segment (start 118.27 106.35) (end 118.27 109.27) (width 0.2) (layer "F.Cu") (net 1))
 (segment (start 118.27 109.27) (end 120.75 111.75) (width 0.2) (layer "F.Cu") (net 1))
 (segment (start 121.65 113.34) (end 121.65 107.65) (width 0.2) (layer "F.Cu") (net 2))
 (segment (start 121.65 107.65) (end 120.5 106.5) (width 0.2) (layer "F.Cu") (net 2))
 (segment (start 120.5 114.49) (end 121.65 113.34) (width 0.2) (layer "F.Cu") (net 2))
 (segment (start 107.55 99.261522) (end 111.511522 95.3) (width 0.2) (layer "F.Cu") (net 3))
 (segment (start 118.629365 101.6) (end 120.65 101.6) (width 0.2) (layer "F.Cu") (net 3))
 (segment (start 117.985 100.5) (end 117.985 100.955635) (width 0.2) (layer "F.Cu") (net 3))
 (segment (start 107.55 103.1) (end 107.55 99.261522) (width 0.2) (layer "F.Cu") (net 3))
 (segment (start 107.55 103.2) (end 107.25 103.5) (width 0.2) (layer "F.Cu") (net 3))
 (segment (start 107.55 96.6) (end 107.55 103.2) (width 0.2) (layer "F.Cu") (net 3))
 (segment (start 117.985 100.955635) (end 118.629365 101.6) (width 0.2) (layer "F.Cu") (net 3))
 (segment (start 120.65 101.6) (end 121.75 100.5) (width 0.2) (layer "F.Cu") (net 3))
 (segment (start 112.785 95.3) (end 117.985 100.5) (width 0.2) (layer "F.Cu") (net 3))
 (segment (start 111.511522 95.3) (end 112.785 95.3) (width 0.2) (layer "F.Cu") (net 3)))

